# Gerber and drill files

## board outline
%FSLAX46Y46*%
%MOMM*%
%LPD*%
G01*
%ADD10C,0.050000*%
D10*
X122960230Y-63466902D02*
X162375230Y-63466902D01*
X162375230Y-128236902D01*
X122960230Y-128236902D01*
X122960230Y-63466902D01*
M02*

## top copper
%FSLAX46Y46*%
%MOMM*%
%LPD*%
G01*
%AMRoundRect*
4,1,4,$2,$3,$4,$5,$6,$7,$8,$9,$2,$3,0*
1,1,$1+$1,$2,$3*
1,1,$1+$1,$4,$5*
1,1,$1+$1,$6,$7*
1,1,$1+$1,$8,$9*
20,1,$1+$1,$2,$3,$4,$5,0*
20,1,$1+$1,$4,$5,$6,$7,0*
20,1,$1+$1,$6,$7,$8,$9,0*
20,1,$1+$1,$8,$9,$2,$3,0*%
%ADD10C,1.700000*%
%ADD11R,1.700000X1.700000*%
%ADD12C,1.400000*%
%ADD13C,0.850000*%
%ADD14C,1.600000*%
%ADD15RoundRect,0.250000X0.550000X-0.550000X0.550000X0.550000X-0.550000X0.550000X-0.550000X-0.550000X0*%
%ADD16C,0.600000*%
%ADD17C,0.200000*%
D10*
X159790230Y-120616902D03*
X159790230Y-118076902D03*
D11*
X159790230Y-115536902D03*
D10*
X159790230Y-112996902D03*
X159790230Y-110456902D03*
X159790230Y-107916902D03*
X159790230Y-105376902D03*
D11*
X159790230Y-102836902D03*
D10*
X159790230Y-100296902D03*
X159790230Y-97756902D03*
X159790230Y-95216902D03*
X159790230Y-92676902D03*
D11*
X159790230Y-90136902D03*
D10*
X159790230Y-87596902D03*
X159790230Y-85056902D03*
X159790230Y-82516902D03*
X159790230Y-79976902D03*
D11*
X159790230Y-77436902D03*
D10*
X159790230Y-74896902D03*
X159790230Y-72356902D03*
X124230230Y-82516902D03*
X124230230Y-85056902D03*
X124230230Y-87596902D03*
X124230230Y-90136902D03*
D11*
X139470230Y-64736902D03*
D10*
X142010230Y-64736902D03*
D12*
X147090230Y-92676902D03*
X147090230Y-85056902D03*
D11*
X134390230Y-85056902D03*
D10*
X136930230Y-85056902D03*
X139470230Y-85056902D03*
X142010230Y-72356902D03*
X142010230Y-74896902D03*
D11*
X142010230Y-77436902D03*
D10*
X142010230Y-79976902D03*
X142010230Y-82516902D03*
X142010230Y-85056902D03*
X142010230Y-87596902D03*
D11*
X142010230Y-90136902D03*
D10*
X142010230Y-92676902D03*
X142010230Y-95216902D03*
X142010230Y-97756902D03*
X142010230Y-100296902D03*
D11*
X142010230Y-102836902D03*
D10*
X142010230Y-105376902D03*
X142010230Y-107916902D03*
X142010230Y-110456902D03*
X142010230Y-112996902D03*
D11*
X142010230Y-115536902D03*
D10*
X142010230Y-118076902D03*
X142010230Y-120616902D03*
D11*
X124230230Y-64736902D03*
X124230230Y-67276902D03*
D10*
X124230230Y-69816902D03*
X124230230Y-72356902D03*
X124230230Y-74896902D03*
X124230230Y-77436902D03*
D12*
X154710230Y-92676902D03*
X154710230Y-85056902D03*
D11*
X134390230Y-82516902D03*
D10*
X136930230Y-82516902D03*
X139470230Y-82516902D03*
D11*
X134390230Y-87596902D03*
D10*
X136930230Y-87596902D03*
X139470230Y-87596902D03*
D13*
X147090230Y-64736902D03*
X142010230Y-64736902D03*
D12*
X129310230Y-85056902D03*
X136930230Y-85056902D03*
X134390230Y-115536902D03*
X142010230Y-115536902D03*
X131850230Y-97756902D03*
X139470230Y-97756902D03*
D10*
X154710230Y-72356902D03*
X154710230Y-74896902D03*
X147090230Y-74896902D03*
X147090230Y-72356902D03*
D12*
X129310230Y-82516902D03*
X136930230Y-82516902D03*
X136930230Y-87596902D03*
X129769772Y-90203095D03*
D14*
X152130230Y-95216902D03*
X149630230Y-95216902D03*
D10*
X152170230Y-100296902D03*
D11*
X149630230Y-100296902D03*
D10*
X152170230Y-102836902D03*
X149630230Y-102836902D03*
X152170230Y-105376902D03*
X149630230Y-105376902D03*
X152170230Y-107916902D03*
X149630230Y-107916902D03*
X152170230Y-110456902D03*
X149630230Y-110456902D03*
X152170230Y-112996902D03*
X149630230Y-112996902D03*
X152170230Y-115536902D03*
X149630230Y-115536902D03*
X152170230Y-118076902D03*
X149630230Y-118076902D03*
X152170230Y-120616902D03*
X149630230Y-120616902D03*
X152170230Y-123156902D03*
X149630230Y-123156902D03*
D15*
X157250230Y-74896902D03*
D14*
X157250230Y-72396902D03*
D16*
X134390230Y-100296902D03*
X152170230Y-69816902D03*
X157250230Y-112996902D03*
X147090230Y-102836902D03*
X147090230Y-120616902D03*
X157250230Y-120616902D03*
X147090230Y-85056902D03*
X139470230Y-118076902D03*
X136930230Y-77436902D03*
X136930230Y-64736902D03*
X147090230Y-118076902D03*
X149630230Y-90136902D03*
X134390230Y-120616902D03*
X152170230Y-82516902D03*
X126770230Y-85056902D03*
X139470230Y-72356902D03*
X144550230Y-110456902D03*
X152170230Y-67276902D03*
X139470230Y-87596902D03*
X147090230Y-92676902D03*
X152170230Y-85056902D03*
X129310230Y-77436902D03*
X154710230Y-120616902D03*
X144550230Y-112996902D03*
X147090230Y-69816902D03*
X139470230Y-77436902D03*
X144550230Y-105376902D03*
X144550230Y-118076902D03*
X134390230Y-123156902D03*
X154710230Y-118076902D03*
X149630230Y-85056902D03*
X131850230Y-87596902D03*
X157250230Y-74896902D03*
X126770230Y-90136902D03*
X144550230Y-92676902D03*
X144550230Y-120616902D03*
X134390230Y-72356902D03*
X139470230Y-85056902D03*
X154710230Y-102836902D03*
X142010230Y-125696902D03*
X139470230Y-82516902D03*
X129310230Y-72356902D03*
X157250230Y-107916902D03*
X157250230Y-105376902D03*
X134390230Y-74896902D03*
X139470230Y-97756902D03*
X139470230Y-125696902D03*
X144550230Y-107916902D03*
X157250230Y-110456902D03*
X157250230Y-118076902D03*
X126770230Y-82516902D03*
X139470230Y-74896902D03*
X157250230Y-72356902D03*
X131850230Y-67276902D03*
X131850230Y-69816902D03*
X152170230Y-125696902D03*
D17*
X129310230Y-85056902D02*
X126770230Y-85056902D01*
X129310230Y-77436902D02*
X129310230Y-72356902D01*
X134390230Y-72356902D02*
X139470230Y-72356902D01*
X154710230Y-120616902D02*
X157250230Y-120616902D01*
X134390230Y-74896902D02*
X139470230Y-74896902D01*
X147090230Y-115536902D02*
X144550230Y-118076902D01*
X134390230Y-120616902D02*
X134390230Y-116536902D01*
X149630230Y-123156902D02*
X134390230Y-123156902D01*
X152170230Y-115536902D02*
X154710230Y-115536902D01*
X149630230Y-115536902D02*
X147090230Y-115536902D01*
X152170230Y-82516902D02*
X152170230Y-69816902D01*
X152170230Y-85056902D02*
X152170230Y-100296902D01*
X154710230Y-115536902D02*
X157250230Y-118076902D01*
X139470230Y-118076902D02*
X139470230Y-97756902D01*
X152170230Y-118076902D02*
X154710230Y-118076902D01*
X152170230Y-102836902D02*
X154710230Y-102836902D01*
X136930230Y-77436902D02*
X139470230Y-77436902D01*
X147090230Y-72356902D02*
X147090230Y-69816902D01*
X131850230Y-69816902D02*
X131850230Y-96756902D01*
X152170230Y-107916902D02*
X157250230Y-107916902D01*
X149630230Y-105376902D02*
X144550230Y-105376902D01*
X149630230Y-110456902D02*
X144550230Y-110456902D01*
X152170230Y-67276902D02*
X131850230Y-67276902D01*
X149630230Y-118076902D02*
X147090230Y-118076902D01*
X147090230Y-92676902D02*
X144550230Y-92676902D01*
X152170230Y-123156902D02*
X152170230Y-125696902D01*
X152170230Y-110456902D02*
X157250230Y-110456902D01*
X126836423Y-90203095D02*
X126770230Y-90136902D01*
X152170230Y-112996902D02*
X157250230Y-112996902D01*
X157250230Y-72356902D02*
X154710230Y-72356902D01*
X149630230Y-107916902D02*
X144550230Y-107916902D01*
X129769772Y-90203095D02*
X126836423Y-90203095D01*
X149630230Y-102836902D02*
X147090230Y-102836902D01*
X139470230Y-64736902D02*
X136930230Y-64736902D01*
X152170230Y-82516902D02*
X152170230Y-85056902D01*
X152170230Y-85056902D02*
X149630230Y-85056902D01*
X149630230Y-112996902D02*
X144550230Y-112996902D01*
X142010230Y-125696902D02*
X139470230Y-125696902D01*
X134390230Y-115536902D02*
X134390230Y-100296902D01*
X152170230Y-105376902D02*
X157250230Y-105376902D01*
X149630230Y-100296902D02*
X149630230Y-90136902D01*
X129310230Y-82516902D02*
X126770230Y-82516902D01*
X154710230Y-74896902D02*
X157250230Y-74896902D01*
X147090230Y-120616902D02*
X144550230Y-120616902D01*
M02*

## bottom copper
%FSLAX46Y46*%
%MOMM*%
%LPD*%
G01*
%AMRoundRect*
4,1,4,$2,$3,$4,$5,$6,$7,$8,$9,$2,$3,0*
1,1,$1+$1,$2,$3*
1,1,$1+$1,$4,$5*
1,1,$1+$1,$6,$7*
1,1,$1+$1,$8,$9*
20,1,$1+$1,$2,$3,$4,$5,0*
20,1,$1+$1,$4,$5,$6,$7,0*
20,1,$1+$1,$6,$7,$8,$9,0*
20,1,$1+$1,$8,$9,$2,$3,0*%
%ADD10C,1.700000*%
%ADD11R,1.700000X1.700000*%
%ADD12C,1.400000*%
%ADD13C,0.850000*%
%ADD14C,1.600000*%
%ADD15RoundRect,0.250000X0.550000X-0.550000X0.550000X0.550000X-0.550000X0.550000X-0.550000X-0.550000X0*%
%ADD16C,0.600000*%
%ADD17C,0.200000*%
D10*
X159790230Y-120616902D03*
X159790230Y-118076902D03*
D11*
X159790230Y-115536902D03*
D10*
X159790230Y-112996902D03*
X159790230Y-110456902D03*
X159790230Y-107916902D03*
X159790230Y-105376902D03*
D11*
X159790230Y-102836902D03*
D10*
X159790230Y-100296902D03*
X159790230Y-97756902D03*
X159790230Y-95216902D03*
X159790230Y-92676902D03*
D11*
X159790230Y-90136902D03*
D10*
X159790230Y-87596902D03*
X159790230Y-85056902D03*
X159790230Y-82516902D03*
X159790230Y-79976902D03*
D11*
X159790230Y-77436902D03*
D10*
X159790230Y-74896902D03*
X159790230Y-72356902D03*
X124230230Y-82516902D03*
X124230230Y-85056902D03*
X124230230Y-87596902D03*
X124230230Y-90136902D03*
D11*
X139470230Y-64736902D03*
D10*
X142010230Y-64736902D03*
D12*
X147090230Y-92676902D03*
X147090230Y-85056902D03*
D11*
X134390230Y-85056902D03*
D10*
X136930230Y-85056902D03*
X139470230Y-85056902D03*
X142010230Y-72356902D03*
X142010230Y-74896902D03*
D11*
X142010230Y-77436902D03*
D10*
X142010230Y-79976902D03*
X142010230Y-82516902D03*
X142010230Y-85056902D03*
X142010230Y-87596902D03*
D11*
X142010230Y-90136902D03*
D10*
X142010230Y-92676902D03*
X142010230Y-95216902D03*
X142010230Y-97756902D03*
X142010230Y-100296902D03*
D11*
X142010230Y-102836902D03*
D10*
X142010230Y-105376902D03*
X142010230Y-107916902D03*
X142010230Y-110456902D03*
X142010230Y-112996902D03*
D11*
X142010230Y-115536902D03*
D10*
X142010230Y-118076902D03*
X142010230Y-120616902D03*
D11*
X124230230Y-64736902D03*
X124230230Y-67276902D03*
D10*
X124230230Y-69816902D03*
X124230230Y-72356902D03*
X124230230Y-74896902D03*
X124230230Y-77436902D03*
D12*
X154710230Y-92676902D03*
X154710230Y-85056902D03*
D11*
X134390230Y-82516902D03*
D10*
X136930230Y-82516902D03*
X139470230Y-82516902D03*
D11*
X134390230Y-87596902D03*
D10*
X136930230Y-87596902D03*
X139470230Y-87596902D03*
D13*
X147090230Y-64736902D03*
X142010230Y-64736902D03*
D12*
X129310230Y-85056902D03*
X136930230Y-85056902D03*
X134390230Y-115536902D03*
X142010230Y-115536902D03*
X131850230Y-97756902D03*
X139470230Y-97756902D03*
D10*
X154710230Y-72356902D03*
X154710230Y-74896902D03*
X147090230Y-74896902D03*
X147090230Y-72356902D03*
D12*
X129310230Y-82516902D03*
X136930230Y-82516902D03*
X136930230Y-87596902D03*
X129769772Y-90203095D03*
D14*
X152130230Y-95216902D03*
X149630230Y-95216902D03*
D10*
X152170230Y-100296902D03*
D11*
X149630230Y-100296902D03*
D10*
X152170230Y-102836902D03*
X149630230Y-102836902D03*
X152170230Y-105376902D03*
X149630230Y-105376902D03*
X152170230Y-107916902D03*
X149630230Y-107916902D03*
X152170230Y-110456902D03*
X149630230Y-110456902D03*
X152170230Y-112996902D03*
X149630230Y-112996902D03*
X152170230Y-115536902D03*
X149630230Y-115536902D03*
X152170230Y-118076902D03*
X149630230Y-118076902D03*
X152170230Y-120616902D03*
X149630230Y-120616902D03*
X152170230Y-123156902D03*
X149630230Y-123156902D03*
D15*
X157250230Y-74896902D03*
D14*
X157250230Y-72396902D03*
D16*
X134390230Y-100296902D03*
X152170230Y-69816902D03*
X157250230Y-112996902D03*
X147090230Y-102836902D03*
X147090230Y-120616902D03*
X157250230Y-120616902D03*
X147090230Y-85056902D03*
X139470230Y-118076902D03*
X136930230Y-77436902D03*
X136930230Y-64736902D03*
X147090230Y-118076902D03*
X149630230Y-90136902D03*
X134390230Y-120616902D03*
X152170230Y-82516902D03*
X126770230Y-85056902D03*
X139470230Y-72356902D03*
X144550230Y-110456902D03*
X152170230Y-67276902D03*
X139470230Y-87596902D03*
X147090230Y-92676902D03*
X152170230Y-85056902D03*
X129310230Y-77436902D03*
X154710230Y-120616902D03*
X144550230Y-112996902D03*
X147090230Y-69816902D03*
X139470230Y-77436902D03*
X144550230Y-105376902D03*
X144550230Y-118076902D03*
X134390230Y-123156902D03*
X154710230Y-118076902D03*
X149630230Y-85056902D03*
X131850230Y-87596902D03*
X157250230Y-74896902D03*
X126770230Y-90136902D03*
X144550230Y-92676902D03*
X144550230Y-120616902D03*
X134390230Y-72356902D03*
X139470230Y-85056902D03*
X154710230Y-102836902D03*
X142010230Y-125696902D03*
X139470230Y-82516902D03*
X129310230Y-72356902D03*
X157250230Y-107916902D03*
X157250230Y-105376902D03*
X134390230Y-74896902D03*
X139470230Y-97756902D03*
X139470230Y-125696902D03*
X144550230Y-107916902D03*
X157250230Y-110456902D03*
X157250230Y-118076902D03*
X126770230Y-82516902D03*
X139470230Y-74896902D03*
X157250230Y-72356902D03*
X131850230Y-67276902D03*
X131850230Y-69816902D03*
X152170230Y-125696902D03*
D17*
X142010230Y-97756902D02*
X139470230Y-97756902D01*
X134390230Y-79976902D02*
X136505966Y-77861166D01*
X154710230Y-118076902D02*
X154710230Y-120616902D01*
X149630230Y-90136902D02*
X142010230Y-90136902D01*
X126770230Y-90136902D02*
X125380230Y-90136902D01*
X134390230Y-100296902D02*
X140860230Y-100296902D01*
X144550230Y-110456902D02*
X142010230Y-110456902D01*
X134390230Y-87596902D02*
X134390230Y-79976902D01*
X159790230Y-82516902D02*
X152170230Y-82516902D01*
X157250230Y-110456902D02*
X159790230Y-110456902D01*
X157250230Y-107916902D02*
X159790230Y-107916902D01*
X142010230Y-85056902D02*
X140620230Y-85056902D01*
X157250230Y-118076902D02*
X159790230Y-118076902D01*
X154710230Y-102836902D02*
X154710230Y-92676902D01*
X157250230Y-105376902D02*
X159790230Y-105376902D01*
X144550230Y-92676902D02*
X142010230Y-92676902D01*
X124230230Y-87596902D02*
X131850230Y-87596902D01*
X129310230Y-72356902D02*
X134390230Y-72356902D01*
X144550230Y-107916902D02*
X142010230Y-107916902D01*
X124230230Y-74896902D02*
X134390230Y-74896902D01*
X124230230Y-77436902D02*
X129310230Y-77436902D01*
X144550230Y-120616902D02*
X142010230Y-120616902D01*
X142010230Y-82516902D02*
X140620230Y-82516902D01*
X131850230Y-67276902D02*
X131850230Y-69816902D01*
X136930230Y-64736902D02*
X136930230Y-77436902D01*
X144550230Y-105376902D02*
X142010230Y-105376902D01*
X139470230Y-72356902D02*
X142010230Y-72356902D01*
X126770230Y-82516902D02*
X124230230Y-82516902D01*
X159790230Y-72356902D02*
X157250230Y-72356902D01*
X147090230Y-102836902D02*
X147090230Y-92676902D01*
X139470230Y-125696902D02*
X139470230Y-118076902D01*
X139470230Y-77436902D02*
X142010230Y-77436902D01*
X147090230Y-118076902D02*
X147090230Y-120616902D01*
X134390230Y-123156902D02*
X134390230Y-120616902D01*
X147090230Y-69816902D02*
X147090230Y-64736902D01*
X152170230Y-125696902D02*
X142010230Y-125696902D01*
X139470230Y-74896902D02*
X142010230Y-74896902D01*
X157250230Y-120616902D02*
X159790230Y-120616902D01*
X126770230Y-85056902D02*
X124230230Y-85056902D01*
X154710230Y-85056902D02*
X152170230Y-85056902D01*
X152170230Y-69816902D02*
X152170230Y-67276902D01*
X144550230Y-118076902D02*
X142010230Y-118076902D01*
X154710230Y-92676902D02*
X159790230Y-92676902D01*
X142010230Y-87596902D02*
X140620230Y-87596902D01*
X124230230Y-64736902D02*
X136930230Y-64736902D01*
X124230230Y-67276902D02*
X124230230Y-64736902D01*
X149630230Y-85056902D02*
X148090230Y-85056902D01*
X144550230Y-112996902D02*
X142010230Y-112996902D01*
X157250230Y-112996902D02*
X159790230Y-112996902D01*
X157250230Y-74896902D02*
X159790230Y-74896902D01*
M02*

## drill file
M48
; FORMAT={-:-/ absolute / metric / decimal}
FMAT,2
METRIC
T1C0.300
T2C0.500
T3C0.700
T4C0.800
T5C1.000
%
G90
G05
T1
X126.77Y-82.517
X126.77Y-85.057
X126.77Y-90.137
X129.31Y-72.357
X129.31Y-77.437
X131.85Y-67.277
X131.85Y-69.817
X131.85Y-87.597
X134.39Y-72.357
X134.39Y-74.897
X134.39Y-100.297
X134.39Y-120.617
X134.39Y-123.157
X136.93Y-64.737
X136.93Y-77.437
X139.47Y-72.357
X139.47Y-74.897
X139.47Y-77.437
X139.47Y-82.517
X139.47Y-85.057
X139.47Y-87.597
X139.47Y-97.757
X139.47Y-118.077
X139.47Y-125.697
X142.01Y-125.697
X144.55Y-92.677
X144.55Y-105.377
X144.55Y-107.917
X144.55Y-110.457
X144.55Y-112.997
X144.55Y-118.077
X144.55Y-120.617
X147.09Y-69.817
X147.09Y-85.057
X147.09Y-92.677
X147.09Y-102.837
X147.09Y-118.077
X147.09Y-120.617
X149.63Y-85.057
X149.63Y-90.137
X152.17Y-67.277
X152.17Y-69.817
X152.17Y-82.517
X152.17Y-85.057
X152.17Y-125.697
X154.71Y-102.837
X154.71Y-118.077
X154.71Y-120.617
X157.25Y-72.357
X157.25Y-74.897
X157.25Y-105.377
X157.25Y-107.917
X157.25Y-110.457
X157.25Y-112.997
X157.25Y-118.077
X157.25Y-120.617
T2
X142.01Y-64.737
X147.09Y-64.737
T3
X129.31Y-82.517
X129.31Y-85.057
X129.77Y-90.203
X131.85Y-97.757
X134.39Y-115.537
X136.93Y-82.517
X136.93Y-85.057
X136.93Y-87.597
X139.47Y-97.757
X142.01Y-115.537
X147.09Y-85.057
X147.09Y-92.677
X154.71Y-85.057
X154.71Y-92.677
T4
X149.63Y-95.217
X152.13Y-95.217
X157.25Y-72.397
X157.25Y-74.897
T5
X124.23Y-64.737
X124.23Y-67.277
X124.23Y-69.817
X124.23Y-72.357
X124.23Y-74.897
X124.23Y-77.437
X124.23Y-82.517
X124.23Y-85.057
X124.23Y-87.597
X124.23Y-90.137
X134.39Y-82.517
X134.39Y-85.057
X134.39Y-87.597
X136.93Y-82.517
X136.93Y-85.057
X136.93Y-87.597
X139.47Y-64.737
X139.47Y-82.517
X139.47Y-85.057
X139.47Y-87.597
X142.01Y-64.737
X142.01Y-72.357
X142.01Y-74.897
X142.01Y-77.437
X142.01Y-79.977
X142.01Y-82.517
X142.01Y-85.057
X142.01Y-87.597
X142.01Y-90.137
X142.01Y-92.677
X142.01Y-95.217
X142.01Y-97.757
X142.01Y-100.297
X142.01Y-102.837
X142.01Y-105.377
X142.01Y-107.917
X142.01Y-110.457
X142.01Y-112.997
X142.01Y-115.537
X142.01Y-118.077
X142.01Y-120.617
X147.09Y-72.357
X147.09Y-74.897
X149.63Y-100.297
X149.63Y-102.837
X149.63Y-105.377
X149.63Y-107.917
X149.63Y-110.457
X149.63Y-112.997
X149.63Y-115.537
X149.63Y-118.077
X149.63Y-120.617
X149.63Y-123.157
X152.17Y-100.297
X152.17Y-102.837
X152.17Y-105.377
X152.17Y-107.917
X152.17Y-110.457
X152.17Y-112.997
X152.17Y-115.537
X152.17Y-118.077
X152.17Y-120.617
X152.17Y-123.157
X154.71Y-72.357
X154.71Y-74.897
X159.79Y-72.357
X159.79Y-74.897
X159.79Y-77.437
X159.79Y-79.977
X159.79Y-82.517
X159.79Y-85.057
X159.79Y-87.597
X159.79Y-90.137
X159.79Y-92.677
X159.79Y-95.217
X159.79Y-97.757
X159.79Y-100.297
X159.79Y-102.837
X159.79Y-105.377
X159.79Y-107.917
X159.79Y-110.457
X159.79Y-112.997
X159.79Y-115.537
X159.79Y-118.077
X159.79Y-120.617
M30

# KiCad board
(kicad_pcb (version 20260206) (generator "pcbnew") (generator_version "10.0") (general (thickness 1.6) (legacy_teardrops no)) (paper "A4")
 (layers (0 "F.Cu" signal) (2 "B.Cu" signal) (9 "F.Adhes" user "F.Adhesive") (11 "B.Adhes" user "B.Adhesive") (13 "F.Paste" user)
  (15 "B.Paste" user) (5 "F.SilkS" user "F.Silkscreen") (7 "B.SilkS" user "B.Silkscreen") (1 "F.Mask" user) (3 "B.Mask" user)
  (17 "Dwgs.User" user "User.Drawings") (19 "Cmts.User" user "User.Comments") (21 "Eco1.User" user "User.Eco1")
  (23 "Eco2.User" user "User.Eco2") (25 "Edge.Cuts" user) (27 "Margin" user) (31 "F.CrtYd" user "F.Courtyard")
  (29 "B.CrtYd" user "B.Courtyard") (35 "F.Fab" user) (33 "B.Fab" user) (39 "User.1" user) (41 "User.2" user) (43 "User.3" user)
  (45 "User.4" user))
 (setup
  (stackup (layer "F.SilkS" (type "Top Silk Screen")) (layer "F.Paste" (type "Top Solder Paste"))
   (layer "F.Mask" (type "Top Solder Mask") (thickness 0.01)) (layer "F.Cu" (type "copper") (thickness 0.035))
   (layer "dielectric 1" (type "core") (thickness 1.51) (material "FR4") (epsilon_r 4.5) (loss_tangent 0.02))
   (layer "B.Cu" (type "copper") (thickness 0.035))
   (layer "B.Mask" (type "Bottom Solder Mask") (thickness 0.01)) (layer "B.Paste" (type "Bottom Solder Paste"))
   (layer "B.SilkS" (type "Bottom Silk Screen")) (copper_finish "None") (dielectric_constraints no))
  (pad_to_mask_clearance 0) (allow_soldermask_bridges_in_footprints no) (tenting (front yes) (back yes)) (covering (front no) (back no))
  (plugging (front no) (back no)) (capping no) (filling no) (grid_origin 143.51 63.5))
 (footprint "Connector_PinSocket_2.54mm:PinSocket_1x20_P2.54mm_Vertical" (layer "F.Cu") (at 159.79023 72.356902)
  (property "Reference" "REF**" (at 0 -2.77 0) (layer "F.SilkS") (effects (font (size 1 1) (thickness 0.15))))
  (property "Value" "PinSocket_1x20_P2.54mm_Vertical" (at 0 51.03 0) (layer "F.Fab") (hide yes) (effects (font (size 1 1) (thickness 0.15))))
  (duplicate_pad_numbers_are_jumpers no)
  (pad "21" thru_hole circle (at 0 48.26) (size 1.7 1.7) (drill 1) (layers "*.Cu" "*.Mask") (remove_unused_layers no))
  (pad "22" thru_hole circle (at 0 45.72) (size 1.7 1.7) (drill 1) (layers "*.Cu" "*.Mask") (remove_unused_layers no))
  (pad "23" thru_hole rect (at 0 43.18) (size 1.7 1.7) (drill 1) (layers "*.Cu" "*.Mask") (remove_unused_layers no)
   (thermal_bridge_angle 45))
  (pad "24" thru_hole circle (at 0 40.64) (size 1.7 1.7) (drill 1) (layers "*.Cu" "*.Mask") (remove_unused_layers no))
  (pad "25" thru_hole circle (at 0 38.1) (size 1.7 1.7) (drill 1) (layers "*.Cu" "*.Mask") (remove_unused_layers no))
  (pad "26" thru_hole circle (at 0 35.56) (size 1.7 1.7) (drill 1) (layers "*.Cu" "*.Mask") (remove_unused_layers no))
  (pad "27" thru_hole circle (at 0 33.02) (size 1.7 1.7) (drill 1) (layers "*.Cu" "*.Mask") (remove_unused_layers no))
  (pad "28" thru_hole rect (at 0 30.48) (size 1.7 1.7) (drill 1) (layers "*.Cu" "*.Mask") (remove_unused_layers no)
   (thermal_bridge_angle 45))
  (pad "29" thru_hole circle (at 0 27.94) (size 1.7 1.7) (drill 1) (layers "*.Cu" "*.Mask") (remove_unused_layers no))
  (pad "30" thru_hole circle (at 0 25.4) (size 1.7 1.7) (drill 1) (layers "*.Cu" "*.Mask") (remove_unused_layers no))
  (pad "31" thru_hole circle (at 0 22.86) (size 1.7 1.7) (drill 1) (layers "*.Cu" "*.Mask") (remove_unused_layers no))
  (pad "32" thru_hole circle (at 0 20.32) (size 1.7 1.7) (drill 1) (layers "*.Cu" "*.Mask") (remove_unused_layers no))
  (pad "33" thru_hole rect (at 0 17.78) (size 1.7 1.7) (drill 1) (layers "*.Cu" "*.Mask") (remove_unused_layers no)
   (thermal_bridge_angle 45))
  (pad "34" thru_hole circle (at 0 15.24) (size 1.7 1.7) (drill 1) (layers "*.Cu" "*.Mask") (remove_unused_layers no))
  (pad "35" thru_hole circle (at 0 12.7) (size 1.7 1.7) (drill 1) (layers "*.Cu" "*.Mask") (remove_unused_layers no))
  (pad "36" thru_hole circle (at 0 10.16) (size 1.7 1.7) (drill 1) (layers "*.Cu" "*.Mask") (remove_unused_layers no))
  (pad "37" thru_hole circle (at 0 7.62) (size 1.7 1.7) (drill 1) (layers "*.Cu" "*.Mask") (remove_unused_layers no))
  (pad "38" thru_hole rect (at 0 5.08) (size 1.7 1.7) (drill 1) (layers "*.Cu" "*.Mask") (remove_unused_layers no) (thermal_bridge_angle 45))
  (pad "39" thru_hole circle (at 0 2.54) (size 1.7 1.7) (drill 1) (layers "*.Cu" "*.Mask") (remove_unused_layers no))
  (pad "40" thru_hole circle (at 0 0) (size 1.7 1.7) (drill 1) (layers "*.Cu" "*.Mask") (remove_unused_layers no) (thermal_bridge_angle 90)))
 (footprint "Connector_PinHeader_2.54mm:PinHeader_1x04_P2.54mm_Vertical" (layer "F.Cu") (at 124.23023 82.516902)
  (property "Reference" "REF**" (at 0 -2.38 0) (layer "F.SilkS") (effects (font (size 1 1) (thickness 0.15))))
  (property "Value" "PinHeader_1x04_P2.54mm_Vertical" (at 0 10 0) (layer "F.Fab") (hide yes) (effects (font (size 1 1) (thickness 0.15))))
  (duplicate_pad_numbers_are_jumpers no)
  (pad "1" thru_hole circle (at 0 0) (size 1.7 1.7) (drill 1) (layers "*.Cu" "*.Mask") (remove_unused_layers no) (thermal_bridge_angle 90))
  (pad "2" thru_hole circle (at 0 2.54) (size 1.7 1.7) (drill 1) (layers "*.Cu" "*.Mask") (remove_unused_layers no))
  (pad "3" thru_hole circle (at 0 5.08) (size 1.7 1.7) (drill 1) (layers "*.Cu" "*.Mask") (remove_unused_layers no))
  (pad "4" thru_hole circle (at 0 7.62) (size 1.7 1.7) (drill 1) (layers "*.Cu" "*.Mask") (remove_unused_layers no)))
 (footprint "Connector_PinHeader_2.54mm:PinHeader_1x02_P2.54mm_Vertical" (layer "F.Cu") (at 139.47023 64.736902 90)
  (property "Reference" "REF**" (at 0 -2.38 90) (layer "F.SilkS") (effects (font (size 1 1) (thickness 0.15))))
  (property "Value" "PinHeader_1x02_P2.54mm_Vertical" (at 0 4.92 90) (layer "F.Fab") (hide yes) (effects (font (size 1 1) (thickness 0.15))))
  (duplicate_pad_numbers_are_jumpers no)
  (pad "1" thru_hole rect (at 0 0 90) (size 1.7 1.7) (drill 1) (layers "*.Cu" "*.Mask") (remove_unused_layers no))
  (pad "2" thru_hole circle (at 0 2.54 90) (size 1.7 1.7) (drill 1) (layers "*.Cu" "*.Mask") (remove_unused_layers no)))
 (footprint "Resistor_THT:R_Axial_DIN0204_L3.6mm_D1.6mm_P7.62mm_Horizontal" (layer "F.Cu") (at 147.09023 92.676902 90)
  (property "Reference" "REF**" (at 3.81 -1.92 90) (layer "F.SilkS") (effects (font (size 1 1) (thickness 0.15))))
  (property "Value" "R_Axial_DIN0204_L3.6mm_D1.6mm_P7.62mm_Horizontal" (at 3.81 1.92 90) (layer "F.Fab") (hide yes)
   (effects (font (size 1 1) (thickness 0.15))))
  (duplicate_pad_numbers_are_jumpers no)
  (pad "1" thru_hole circle (at 0 0 90) (size 1.4 1.4) (drill 0.7) (layers "*.Cu" "*.Mask") (remove_unused_layers no))
  (pad "2" thru_hole circle (at 7.62 0 90) (size 1.4 1.4) (drill 0.7) (layers "*.Cu" "*.Mask") (remove_unused_layers no)))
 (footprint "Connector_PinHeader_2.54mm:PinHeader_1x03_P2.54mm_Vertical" (layer "F.Cu") (at 134.39023 85.056902 90)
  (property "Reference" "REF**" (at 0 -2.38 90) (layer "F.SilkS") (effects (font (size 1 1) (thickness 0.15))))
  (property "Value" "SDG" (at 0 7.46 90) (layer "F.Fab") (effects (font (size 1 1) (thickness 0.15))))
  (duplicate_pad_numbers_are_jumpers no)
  (pad "1" thru_hole rect (at 0 0 90) (size 1.7 1.7) (drill 1) (layers "*.Cu" "*.Mask") (remove_unused_layers no))
  (pad "2" thru_hole circle (at 0 2.54 90) (size 1.7 1.7) (drill 1) (layers "*.Cu" "*.Mask") (remove_unused_layers no))
  (pad "3" thru_hole circle (at 0 5.08 90) (size 1.7 1.7) (drill 1) (layers "*.Cu" "*.Mask") (remove_unused_layers no)))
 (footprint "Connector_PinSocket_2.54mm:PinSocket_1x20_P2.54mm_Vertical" (layer "F.Cu") (at 142.01023 72.356902)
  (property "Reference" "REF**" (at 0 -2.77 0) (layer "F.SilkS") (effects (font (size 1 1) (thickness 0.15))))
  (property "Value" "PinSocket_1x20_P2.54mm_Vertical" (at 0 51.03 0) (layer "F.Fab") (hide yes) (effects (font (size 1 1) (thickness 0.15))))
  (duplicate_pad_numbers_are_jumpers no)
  (pad "1" thru_hole circle (at 0 0) (size 1.7 1.7) (drill 1) (layers "*.Cu" "*.Mask") (remove_unused_layers no) (thermal_bridge_angle 90))
  (pad "2" thru_hole circle (at 0 2.54) (size 1.7 1.7) (drill 1) (layers "*.Cu" "*.Mask") (remove_unused_layers no))
  (pad "3" thru_hole rect (at 0 5.08) (size 1.7 1.7) (drill 1) (layers "*.Cu" "*.Mask") (remove_unused_layers no) (thermal_bridge_angle 45))
  (pad "4" thru_hole circle (at 0 7.62) (size 1.7 1.7) (drill 1) (layers "*.Cu" "*.Mask") (remove_unused_layers no))
  (pad "5" thru_hole circle (at 0 10.16) (size 1.7 1.7) (drill 1) (layers "*.Cu" "*.Mask") (remove_unused_layers no))
  (pad "6" thru_hole circle (at 0 12.7) (size 1.7 1.7) (drill 1) (layers "*.Cu" "*.Mask") (remove_unused_layers no))
  (pad "7" thru_hole circle (at 0 15.24) (size 1.7 1.7) (drill 1) (layers "*.Cu" "*.Mask") (remove_unused_layers no))
  (pad "8" thru_hole rect (at 0 17.78) (size 1.7 1.7) (drill 1) (layers "*.Cu" "*.Mask") (remove_unused_layers no) (thermal_bridge_angle 45))
  (pad "9" thru_hole circle (at 0 20.32) (size 1.7 1.7) (drill 1) (layers "*.Cu" "*.Mask") (remove_unused_layers no))
  (pad "10" thru_hole circle (at 0 22.86) (size 1.7 1.7) (drill 1) (layers "*.Cu" "*.Mask") (remove_unused_layers no))
  (pad "11" thru_hole circle (at 0 25.4) (size 1.7 1.7) (drill 1) (layers "*.Cu" "*.Mask") (remove_unused_layers no))
  (pad "12" thru_hole circle (at 0 27.94) (size 1.7 1.7) (drill 1) (layers "*.Cu" "*.Mask") (remove_unused_layers no))
  (pad "13" thru_hole rect (at 0 30.48) (size 1.7 1.7) (drill 1) (layers "*.Cu" "*.Mask") (remove_unused_layers no)
   (thermal_bridge_angle 45))
  (pad "14" thru_hole circle (at 0 33.02) (size 1.7 1.7) (drill 1) (layers "*.Cu" "*.Mask") (remove_unused_layers no))
  (pad "15" thru_hole circle (at 0 35.56) (size 1.7 1.7) (drill 1) (layers "*.Cu" "*.Mask") (remove_unused_layers no))
  (pad "16" thru_hole circle (at 0 38.1) (size 1.7 1.7) (drill 1) (layers "*.Cu" "*.Mask") (remove_unused_layers no))
  (pad "17" thru_hole circle (at 0 40.64) (size 1.7 1.7) (drill 1) (layers "*.Cu" "*.Mask") (remove_unused_layers no))
  (pad "18" thru_hole rect (at 0 43.18) (size 1.7 1.7) (drill 1) (layers "*.Cu" "*.Mask") (remove_unused_layers no)
   (thermal_bridge_angle 45))
  (pad "19" thru_hole circle (at 0 45.72) (size 1.7 1.7) (drill 1) (layers "*.Cu" "*.Mask") (remove_unused_layers no))
  (pad "20" thru_hole circle (at 0 48.26) (size 1.7 1.7) (drill 1) (layers "*.Cu" "*.Mask") (remove_unused_layers no)))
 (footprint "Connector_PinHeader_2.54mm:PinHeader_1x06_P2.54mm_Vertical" (layer "F.Cu") (at 124.23023 64.736902)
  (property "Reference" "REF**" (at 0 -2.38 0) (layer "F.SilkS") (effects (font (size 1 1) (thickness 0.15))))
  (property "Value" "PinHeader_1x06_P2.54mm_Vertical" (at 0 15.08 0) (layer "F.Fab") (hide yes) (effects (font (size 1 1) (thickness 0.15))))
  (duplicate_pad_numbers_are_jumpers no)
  (pad "1" thru_hole rect (at 0 0) (size 1.7 1.7) (drill 1) (layers "*.Cu" "*.Mask") (remove_unused_layers no))
  (pad "2" thru_hole rect (at 0 2.54) (size 1.7 1.7) (drill 1) (layers "*.Cu" "*.Mask") (remove_unused_layers no) (thermal_bridge_angle 45))
  (pad "3" thru_hole circle (at 0 5.08) (size 1.7 1.7) (drill 1) (layers "*.Cu" "*.Mask") (remove_unused_layers no))
  (pad "4" thru_hole circle (at 0 7.62) (size 1.7 1.7) (drill 1) (layers "*.Cu" "*.Mask") (remove_unused_layers no))
  (pad "5" thru_hole circle (at 0 10.16) (size 1.7 1.7) (drill 1) (layers "*.Cu" "*.Mask") (remove_unused_layers no))
  (pad "6" thru_hole circle (at 0 12.7) (size 1.7 1.7) (drill 1) (layers "*.Cu" "*.Mask") (remove_unused_layers no)))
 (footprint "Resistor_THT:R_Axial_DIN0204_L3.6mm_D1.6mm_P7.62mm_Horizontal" (layer "F.Cu") (at 154.71023 92.676902 90)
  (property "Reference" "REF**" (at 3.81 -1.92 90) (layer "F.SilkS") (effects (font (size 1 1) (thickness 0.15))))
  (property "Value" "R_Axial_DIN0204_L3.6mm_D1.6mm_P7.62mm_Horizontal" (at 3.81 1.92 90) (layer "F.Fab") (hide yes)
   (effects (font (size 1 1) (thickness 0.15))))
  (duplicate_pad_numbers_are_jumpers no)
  (pad "1" thru_hole circle (at 0 0 90) (size 1.4 1.4) (drill 0.7) (layers "*.Cu" "*.Mask") (remove_unused_layers no))
  (pad "2" thru_hole circle (at 7.62 0 90) (size 1.4 1.4) (drill 0.7) (layers "*.Cu" "*.Mask") (remove_unused_layers no)))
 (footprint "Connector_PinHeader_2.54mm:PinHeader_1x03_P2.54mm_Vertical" (layer "F.Cu") (at 134.39023 82.516902 90)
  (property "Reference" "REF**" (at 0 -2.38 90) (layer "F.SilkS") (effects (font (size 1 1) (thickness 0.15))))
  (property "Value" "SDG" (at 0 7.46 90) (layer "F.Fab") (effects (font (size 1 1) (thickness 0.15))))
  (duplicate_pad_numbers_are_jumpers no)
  (pad "1" thru_hole rect (at 0 0 90) (size 1.7 1.7) (drill 1) (layers "*.Cu" "*.Mask") (remove_unused_layers no))
  (pad "2" thru_hole circle (at 0 2.54 90) (size 1.7 1.7) (drill 1) (layers "*.Cu" "*.Mask") (remove_unused_layers no))
  (pad "3" thru_hole circle (at 0 5.08 90) (size 1.7 1.7) (drill 1) (layers "*.Cu" "*.Mask") (remove_unused_layers no)))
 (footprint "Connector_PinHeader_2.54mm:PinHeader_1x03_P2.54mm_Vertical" (layer "F.Cu") (at 134.39023 87.596902 90)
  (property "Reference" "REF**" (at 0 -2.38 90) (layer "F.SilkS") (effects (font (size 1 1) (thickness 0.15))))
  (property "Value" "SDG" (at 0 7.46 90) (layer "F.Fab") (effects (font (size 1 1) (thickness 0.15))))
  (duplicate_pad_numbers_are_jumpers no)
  (pad "1" thru_hole rect (at 0 0 90) (size 1.7 1.7) (drill 1) (layers "*.Cu" "*.Mask") (remove_unused_layers no))
  (pad "2" thru_hole circle (at 0 2.54 90) (size 1.7 1.7) (drill 1) (layers "*.Cu" "*.Mask") (remove_unused_layers no))
  (pad "3" thru_hole circle (at 0 5.08 90) (size 1.7 1.7) (drill 1) (layers "*.Cu" "*.Mask") (remove_unused_layers no)))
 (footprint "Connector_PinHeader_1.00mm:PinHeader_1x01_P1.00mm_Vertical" (layer "B.Cu") (at 147.09023 64.736902 180)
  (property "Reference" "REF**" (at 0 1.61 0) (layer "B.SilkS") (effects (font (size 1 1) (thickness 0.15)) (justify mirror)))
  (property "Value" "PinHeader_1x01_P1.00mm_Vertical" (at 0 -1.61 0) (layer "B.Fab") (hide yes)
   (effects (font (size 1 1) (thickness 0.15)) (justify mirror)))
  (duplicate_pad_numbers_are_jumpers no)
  (pad "1" thru_hole circle (at 0 0 180) (size 0.85 0.85) (drill 0.5) (layers "*.Cu" "*.Mask") (remove_unused_layers no)
   (thermal_bridge_angle 90))
  (pad "2" thru_hole circle (at 5.08 0 180) (size 0.85 0.85) (drill 0.5) (layers "*.Cu" "*.Mask") (remove_unused_layers no)
   (thermal_bridge_angle 90)))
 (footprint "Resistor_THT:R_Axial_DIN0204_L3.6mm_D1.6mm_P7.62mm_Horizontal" (layer "B.Cu") (at 129.31023 85.056902)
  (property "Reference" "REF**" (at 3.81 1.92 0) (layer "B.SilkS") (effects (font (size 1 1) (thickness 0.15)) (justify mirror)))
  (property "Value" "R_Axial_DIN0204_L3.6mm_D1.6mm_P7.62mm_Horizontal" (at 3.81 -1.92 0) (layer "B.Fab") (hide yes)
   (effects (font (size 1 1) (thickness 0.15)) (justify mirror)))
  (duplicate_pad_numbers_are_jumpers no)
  (pad "1" thru_hole circle (at 0 0) (size 1.4 1.4) (drill 0.7) (layers "*.Cu" "*.Mask") (remove_unused_layers no))
  (pad "2" thru_hole circle (at 7.62 0) (size 1.4 1.4) (drill 0.7) (layers "*.Cu" "*.Mask") (remove_unused_layers no)))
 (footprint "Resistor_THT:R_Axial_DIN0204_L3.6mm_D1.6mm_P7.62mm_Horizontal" (layer "B.Cu") (at 134.39023 115.536902)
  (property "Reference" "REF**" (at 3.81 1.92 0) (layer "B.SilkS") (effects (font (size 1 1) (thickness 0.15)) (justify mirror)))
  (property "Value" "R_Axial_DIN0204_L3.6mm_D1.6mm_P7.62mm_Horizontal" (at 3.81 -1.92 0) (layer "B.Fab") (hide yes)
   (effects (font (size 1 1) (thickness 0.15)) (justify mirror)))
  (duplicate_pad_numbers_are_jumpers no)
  (pad "1" thru_hole circle (at 0 0) (size 1.4 1.4) (drill 0.7) (layers "*.Cu" "*.Mask") (remove_unused_layers no))
  (pad "2" thru_hole circle (at 7.62 0) (size 1.4 1.4) (drill 0.7) (layers "*.Cu" "*.Mask") (remove_unused_layers no)))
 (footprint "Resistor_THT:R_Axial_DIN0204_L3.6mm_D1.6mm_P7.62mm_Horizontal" (layer "B.Cu") (at 131.85023 97.756902)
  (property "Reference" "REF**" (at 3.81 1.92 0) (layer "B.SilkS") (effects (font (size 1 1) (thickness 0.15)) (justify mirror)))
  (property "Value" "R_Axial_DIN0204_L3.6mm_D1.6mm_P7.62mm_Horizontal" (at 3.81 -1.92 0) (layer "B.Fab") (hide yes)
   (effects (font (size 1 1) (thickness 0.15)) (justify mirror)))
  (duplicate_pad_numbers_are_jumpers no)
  (pad "1" thru_hole circle (at 0 0) (size 1.4 1.4) (drill 0.7) (layers "*.Cu" "*.Mask") (remove_unused_layers no))
  (pad "2" thru_hole circle (at 7.62 0) (size 1.4 1.4) (drill 0.7) (layers "*.Cu" "*.Mask") (remove_unused_layers no)))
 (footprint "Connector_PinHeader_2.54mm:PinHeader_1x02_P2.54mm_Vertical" (layer "B.Cu") (at 154.71023 72.356902 180)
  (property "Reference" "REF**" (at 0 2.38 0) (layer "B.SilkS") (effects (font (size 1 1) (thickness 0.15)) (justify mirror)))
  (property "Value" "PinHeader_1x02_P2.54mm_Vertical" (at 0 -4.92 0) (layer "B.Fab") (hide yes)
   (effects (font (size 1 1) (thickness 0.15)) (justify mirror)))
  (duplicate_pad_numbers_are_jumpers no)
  (pad "1" thru_hole circle (at 0 0 180) (size 1.7 1.7) (drill 1) (layers "*.Cu" "*.Mask") (remove_unused_layers no)
   (thermal_bridge_angle 90))
  (pad "2" thru_hole circle (at 0 -2.54 180) (size 1.7 1.7) (drill 1) (layers "*.Cu" "*.Mask") (remove_unused_layers no))
  (pad "3" thru_hole circle (at 7.62 -2.54 180) (size 1.7 1.7) (drill 1) (layers "*.Cu" "*.Mask") (remove_unused_layers no))
  (pad "3" thru_hole circle (at 7.62 0 180) (size 1.7 1.7) (drill 1) (layers "*.Cu" "*.Mask") (remove_unused_layers no)
   (thermal_bridge_angle 90)))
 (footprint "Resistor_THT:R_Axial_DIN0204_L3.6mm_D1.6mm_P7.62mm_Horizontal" (layer "B.Cu") (at 129.31023 82.516902)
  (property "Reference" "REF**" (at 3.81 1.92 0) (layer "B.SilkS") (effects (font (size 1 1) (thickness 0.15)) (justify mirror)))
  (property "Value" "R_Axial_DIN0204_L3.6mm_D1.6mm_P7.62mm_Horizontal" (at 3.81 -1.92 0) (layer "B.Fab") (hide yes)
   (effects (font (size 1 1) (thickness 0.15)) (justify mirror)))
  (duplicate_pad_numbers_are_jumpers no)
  (pad "1" thru_hole circle (at 0 0) (size 1.4 1.4) (drill 0.7) (layers "*.Cu" "*.Mask") (remove_unused_layers no))
  (pad "2" thru_hole circle (at 7.62 0) (size 1.4 1.4) (drill 0.7) (layers "*.Cu" "*.Mask") (remove_unused_layers no)))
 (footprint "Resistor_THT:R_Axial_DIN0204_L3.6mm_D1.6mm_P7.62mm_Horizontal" (layer "B.Cu") (at 136.93023 87.596902 -160)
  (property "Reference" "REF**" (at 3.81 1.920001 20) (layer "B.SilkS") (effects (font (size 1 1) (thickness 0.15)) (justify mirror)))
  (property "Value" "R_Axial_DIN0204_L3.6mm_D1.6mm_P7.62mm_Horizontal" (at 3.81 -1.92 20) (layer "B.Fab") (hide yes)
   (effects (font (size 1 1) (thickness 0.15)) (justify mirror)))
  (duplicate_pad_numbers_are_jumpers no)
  (pad "1" thru_hole circle (at 0 0 200) (size 1.4 1.4) (drill 0.7) (layers "*.Cu" "*.Mask") (remove_unused_layers no))
  (pad "2" thru_hole circle (at 7.62 0.000001 200) (size 1.4 1.4) (drill 0.7) (layers "*.Cu" "*.Mask") (remove_unused_layers no)))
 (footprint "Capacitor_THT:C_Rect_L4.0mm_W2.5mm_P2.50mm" (layer "B.Cu") (at 152.13023 95.216902 180)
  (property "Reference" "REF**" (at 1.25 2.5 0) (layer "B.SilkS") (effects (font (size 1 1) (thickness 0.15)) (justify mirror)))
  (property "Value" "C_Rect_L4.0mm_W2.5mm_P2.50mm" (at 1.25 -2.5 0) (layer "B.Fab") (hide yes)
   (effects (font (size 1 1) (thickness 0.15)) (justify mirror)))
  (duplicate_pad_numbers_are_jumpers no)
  (pad "1" thru_hole circle (at 0 0 180) (size 1.6 1.6) (drill 0.8) (layers "*.Cu" "*.Mask") (remove_unused_layers no))
  (pad "2" thru_hole circle (at 2.5 0 180) (size 1.6 1.6) (drill 0.8) (layers "*.Cu" "*.Mask") (remove_unused_layers no)))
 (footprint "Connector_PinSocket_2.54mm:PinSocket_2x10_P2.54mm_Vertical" (layer "B.Cu") (at 149.63023 100.296902 180)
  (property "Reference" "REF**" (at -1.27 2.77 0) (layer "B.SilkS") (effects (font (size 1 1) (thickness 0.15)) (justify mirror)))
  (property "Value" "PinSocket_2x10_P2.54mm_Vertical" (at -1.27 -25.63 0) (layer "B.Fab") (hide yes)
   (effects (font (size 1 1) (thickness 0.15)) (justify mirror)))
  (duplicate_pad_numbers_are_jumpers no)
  (pad "1" thru_hole circle (at -2.54 0 180) (size 1.7 1.7) (drill 1) (layers "*.Cu" "*.Mask") (remove_unused_layers no))
  (pad "2" thru_hole rect (at 0 0 180) (size 1.7 1.7) (drill 1) (layers "*.Cu" "*.Mask") (remove_unused_layers no))
  (pad "3" thru_hole circle (at -2.54 -2.54 180) (size 1.7 1.7) (drill 1) (layers "*.Cu" "*.Mask") (remove_unused_layers no))
  (pad "4" thru_hole circle (at 0 -2.54 180) (size 1.7 1.7) (drill 1) (layers "*.Cu" "*.Mask") (remove_unused_layers no))
  (pad "5" thru_hole circle (at -2.54 -5.08 180) (size 1.7 1.7) (drill 1) (layers "*.Cu" "*.Mask") (remove_unused_layers no))
  (pad "6" thru_hole circle (at 0 -5.08 180) (size 1.7 1.7) (drill 1) (layers "*.Cu" "*.Mask") (remove_unused_layers no))
  (pad "7" thru_hole circle (at -2.54 -7.62 180) (size 1.7 1.7) (drill 1) (layers "*.Cu" "*.Mask") (remove_unused_layers no))
  (pad "8" thru_hole circle (at 0 -7.62 180) (size 1.7 1.7) (drill 1) (layers "*.Cu" "*.Mask") (remove_unused_layers no))
  (pad "9" thru_hole circle (at -2.54 -10.16 180) (size 1.7 1.7) (drill 1) (layers "*.Cu" "*.Mask") (remove_unused_layers no))
  (pad "10" thru_hole circle (at 0 -10.16 180) (size 1.7 1.7) (drill 1) (layers "*.Cu" "*.Mask") (remove_unused_layers no))
  (pad "11" thru_hole circle (at -2.54 -12.7 180) (size 1.7 1.7) (drill 1) (layers "*.Cu" "*.Mask") (remove_unused_layers no))
  (pad "12" thru_hole circle (at 0 -12.7 180) (size 1.7 1.7) (drill 1) (layers "*.Cu" "*.Mask") (remove_unused_layers no))
  (pad "13" thru_hole circle (at -2.54 -15.24 180) (size 1.7 1.7) (drill 1) (layers "*.Cu" "*.Mask") (remove_unused_layers no))
  (pad "14" thru_hole circle (at 0 -15.24 180) (size 1.7 1.7) (drill 1) (layers "*.Cu" "*.Mask") (remove_unused_layers no))
  (pad "15" thru_hole circle (at -2.54 -17.78 180) (size 1.7 1.7) (drill 1) (layers "*.Cu" "*.Mask") (remove_unused_layers no))
  (pad "16" thru_hole circle (at 0 -17.78 180) (size 1.7 1.7) (drill 1) (layers "*.Cu" "*.Mask") (remove_unused_layers no))
  (pad "17" thru_hole circle (at -2.54 -20.32 180) (size 1.7 1.7) (drill 1) (layers "*.Cu" "*.Mask") (remove_unused_layers no))
  (pad "18" thru_hole circle (at 0 -20.32 180) (size 1.7 1.7) (drill 1) (layers "*.Cu" "*.Mask") (remove_unused_layers no))
  (pad "19" thru_hole circle (at -2.54 -22.86 180) (size 1.7 1.7) (drill 1) (layers "*.Cu" "*.Mask") (remove_unused_layers no))
  (pad "20" thru_hole circle (at 0 -22.86 180) (size 1.7 1.7) (drill 1) (layers "*.Cu" "*.Mask") (remove_unused_layers no)))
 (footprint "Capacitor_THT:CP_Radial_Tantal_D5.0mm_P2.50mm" (layer "B.Cu") (at 157.25023 74.896902 90)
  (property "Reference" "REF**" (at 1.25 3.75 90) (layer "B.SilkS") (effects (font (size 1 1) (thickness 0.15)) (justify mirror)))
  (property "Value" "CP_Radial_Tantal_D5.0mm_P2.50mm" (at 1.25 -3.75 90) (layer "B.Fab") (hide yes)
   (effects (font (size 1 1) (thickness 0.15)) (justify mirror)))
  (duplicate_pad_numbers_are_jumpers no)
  (pad "1" thru_hole roundrect (at 0 0 90) (size 1.6 1.6) (drill 0.8) (layers "*.Cu" "*.Mask") (remove_unused_layers no)
   (roundrect_rratio 0.15625))
  (pad "2" thru_hole circle (at 2.5 0 90) (size 1.6 1.6) (drill 0.8) (layers "*.Cu" "*.Mask") (remove_unused_layers no)))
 (gr_rect (start 122.96023 63.466902) (end 162.37523 128.236902) (stroke (width 0.05) (type solid)) (fill no) (layer "Edge.Cuts"))
 (segment (start 129.31023 85.056902) (end 126.77023 85.056902) (width 0.2) (layer "F.Cu") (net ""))
 (segment (start 129.31023 77.436902) (end 129.31023 72.356902) (width 0.2) (layer "F.Cu") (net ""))
 (segment (start 134.39023 72.356902) (end 139.47023 72.356902) (width 0.2) (layer "F.Cu") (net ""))
 (segment (start 154.71023 120.616902) (end 157.25023 120.616902) (width 0.2) (layer "F.Cu") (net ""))
 (segment (start 134.39023 74.896902) (end 139.47023 74.896902) (width 0.2) (layer "F.Cu") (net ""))
 (segment (start 147.09023 115.536902) (end 144.55023 118.076902) (width 0.2) (layer "F.Cu") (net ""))
 (segment (start 134.39023 120.616902) (end 134.39023 116.536902) (width 0.2) (layer "F.Cu") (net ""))
 (segment (start 149.63023 123.156902) (end 134.39023 123.156902) (width 0.2) (layer "F.Cu") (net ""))
 (segment (start 152.17023 115.536902) (end 154.71023 115.536902) (width 0.2) (layer "F.Cu") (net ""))
 (segment (start 149.63023 115.536902) (end 147.09023 115.536902) (width 0.2) (layer "F.Cu") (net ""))
 (segment (start 152.17023 82.516902) (end 152.17023 69.816902) (width 0.2) (layer "F.Cu") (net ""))
 (segment (start 152.17023 85.056902) (end 152.17023 100.296902) (width 0.2) (layer "F.Cu") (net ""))
 (segment (start 154.71023 115.536902) (end 157.25023 118.076902) (width 0.2) (layer "F.Cu") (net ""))
 (segment (start 139.47023 118.076902) (end 139.47023 97.756902) (width 0.2) (layer "F.Cu") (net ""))
 (segment (start 152.17023 118.076902) (end 154.71023 118.076902) (width 0.2) (layer "F.Cu") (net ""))
 (segment (start 152.17023 102.836902) (end 154.71023 102.836902) (width 0.2) (layer "F.Cu") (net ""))
 (segment (start 136.93023 77.436902) (end 139.47023 77.436902) (width 0.2) (layer "F.Cu") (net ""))
 (segment (start 147.09023 72.356902) (end 147.09023 69.816902) (width 0.2) (layer "F.Cu") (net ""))
 (segment (start 131.85023 69.816902) (end 131.85023 96.756902) (width 0.2) (layer "F.Cu") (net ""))
 (segment (start 152.17023 107.916902) (end 157.25023 107.916902) (width 0.2) (layer "F.Cu") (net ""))
 (segment (start 149.63023 105.376902) (end 144.55023 105.376902) (width 0.2) (layer "F.Cu") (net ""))
 (segment (start 149.63023 110.456902) (end 144.55023 110.456902) (width 0.2) (layer "F.Cu") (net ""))
 (segment (start 152.17023 67.276902) (end 131.85023 67.276902) (width 0.2) (layer "F.Cu") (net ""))
 (segment (start 149.63023 118.076902) (end 147.09023 118.076902) (width 0.2) (layer "F.Cu") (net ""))
 (segment (start 147.09023 92.676902) (end 144.55023 92.676902) (width 0.2) (layer "F.Cu") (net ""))
 (segment (start 152.17023 123.156902) (end 152.17023 125.696902) (width 0.2) (layer "F.Cu") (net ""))
 (segment (start 152.17023 110.456902) (end 157.25023 110.456902) (width 0.2) (layer "F.Cu") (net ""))
 (segment (start 126.836423 90.203095) (end 126.77023 90.136902) (width 0.2) (layer "F.Cu") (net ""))
 (segment (start 152.17023 112.996902) (end 157.25023 112.996902) (width 0.2) (layer "F.Cu") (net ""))
 (segment (start 157.25023 72.356902) (end 154.71023 72.356902) (width 0.2) (layer "F.Cu") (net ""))
 (segment (start 149.63023 107.916902) (end 144.55023 107.916902) (width 0.2) (layer "F.Cu") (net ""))
 (segment (start 129.769772 90.203095) (end 126.836423 90.203095) (width 0.2) (layer "F.Cu") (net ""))
 (segment (start 149.63023 102.836902) (end 147.09023 102.836902) (width 0.2) (layer "F.Cu") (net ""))
 (segment (start 139.47023 64.736902) (end 136.93023 64.736902) (width 0.2) (layer "F.Cu") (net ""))
 (segment (start 152.17023 82.516902) (end 152.17023 85.056902) (width 0.2) (layer "F.Cu") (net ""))
 (segment (start 152.17023 85.056902) (end 149.63023 85.056902) (width 0.2) (layer "F.Cu") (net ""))
 (segment (start 149.63023 112.996902) (end 144.55023 112.996902) (width 0.2) (layer "F.Cu") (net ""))
 (segment (start 142.01023 125.696902) (end 139.47023 125.696902) (width 0.2) (layer "F.Cu") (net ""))
 (segment (start 134.39023 115.536902) (end 134.39023 100.296902) (width 0.2) (layer "F.Cu") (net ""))
 (segment (start 152.17023 105.376902) (end 157.25023 105.376902) (width 0.2) (layer "F.Cu") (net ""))
 (segment (start 149.63023 100.296902) (end 149.63023 90.136902) (width 0.2) (layer "F.Cu") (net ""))
 (segment (start 129.31023 82.516902) (end 126.77023 82.516902) (width 0.2) (layer "F.Cu") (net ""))
 (segment (start 154.71023 74.896902) (end 157.25023 74.896902) (width 0.2) (layer "F.Cu") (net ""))
 (segment (start 147.09023 120.616902) (end 144.55023 120.616902) (width 0.2) (layer "F.Cu") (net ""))
 (via (at 134.39023 100.296902) (size 0.6) (drill 0.3) (layers "F.Cu" "B.Cu") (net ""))
 (via (at 152.17023 69.816902) (size 0.6) (drill 0.3) (layers "F.Cu" "B.Cu") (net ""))
 (via (at 157.25023 112.996902) (size 0.6) (drill 0.3) (layers "F.Cu" "B.Cu") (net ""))
 (via (at 147.09023 102.836902) (size 0.6) (drill 0.3) (layers "F.Cu" "B.Cu") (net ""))
 (via (at 147.09023 120.616902) (size 0.6) (drill 0.3) (layers "F.Cu" "B.Cu") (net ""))
 (via (at 157.25023 120.616902) (size 0.6) (drill 0.3) (layers "F.Cu" "B.Cu") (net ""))
 (via (at 147.09023 85.056902) (size 0.6) (drill 0.3) (layers "F.Cu" "B.Cu") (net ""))
 (via (at 139.47023 118.076902) (size 0.6) (drill 0.3) (layers "F.Cu" "B.Cu") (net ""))
 (via (at 136.93023 77.436902) (size 0.6) (drill 0.3) (layers "F.Cu" "B.Cu") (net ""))
 (via (at 136.93023 64.736902) (size 0.6) (drill 0.3) (layers "F.Cu" "B.Cu") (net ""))
 (via (at 147.09023 118.076902) (size 0.6) (drill 0.3) (layers "F.Cu" "B.Cu") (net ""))
 (via (at 149.63023 90.136902) (size 0.6) (drill 0.3) (layers "F.Cu" "B.Cu") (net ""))
 (via (at 134.39023 120.616902) (size 0.6) (drill 0.3) (layers "F.Cu" "B.Cu") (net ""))
 (via (at 152.17023 82.516902) (size 0.6) (drill 0.3) (layers "F.Cu" "B.Cu") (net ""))
 (via (at 126.77023 85.056902) (size 0.6) (drill 0.3) (layers "F.Cu" "B.Cu") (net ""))
 (via (at 139.47023 72.356902) (size 0.6) (drill 0.3) (layers "F.Cu" "B.Cu") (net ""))
 (via (at 144.55023 110.456902) (size 0.6) (drill 0.3) (layers "F.Cu" "B.Cu") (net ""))
 (via (at 152.17023 67.276902) (size 0.6) (drill 0.3) (layers "F.Cu" "B.Cu") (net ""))
 (via (at 139.47023 87.596902) (size 0.6) (drill 0.3) (layers "F.Cu" "B.Cu") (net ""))
 (via (at 147.09023 92.676902) (size 0.6) (drill 0.3) (layers "F.Cu" "B.Cu") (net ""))
 (via (at 152.17023 85.056902) (size 0.6) (drill 0.3) (layers "F.Cu" "B.Cu") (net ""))
 (via (at 129.31023 77.436902) (size 0.6) (drill 0.3) (layers "F.Cu" "B.Cu") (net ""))
 (via (at 154.71023 120.616902) (size 0.6) (drill 0.3) (layers "F.Cu" "B.Cu") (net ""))
 (via (at 144.55023 112.996902) (size 0.6) (drill 0.3) (layers "F.Cu" "B.Cu") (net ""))
 (via (at 147.09023 69.816902) (size 0.6) (drill 0.3) (layers "F.Cu" "B.Cu") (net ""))
 (via (at 139.47023 77.436902) (size 0.6) (drill 0.3) (layers "F.Cu" "B.Cu") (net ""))
 (via (at 144.55023 105.376902) (size 0.6) (drill 0.3) (layers "F.Cu" "B.Cu") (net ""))
 (via (at 144.55023 118.076902) (size 0.6) (drill 0.3) (layers "F.Cu" "B.Cu") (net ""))
 (via (at 134.39023 123.156902) (size 0.6) (drill 0.3) (layers "F.Cu" "B.Cu") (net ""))
 (via (at 154.71023 118.076902) (size 0.6) (drill 0.3) (layers "F.Cu" "B.Cu") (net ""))
 (via (at 149.63023 85.056902) (size 0.6) (drill 0.3) (layers "F.Cu" "B.Cu") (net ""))
 (via (at 131.85023 87.596902) (size 0.6) (drill 0.3) (layers "F.Cu" "B.Cu") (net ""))
 (via (at 157.25023 74.896902) (size 0.6) (drill 0.3) (layers "F.Cu" "B.Cu") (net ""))
 (via (at 126.77023 90.136902) (size 0.6) (drill 0.3) (layers "F.Cu" "B.Cu") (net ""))
 (via (at 144.55023 92.676902) (size 0.6) (drill 0.3) (layers "F.Cu" "B.Cu") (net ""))
 (via (at 144.55023 120.616902) (size 0.6) (drill 0.3) (layers "F.Cu" "B.Cu") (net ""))
 (via (at 134.39023 72.356902) (size 0.6) (drill 0.3) (layers "F.Cu" "B.Cu") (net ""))
 (via (at 139.47023 85.056902) (size 0.6) (drill 0.3) (layers "F.Cu" "B.Cu") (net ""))
 (via (at 154.71023 102.836902) (size 0.6) (drill 0.3) (layers "F.Cu" "B.Cu") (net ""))
 (via (at 142.01023 125.696902) (size 0.6) (drill 0.3) (layers "F.Cu" "B.Cu") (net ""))
 (via (at 139.47023 82.516902) (size 0.6) (drill 0.3) (layers "F.Cu" "B.Cu") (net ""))
 (via (at 129.31023 72.356902) (size 0.6) (drill 0.3) (layers "F.Cu" "B.Cu") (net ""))
 (via (at 157.25023 107.916902) (size 0.6) (drill 0.3) (layers "F.Cu" "B.Cu") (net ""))
 (via (at 157.25023 105.376902) (size 0.6) (drill 0.3) (layers "F.Cu" "B.Cu") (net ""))
 (via (at 134.39023 74.896902) (size 0.6) (drill 0.3) (layers "F.Cu" "B.Cu") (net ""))
 (via (at 139.47023 97.756902) (size 0.6) (drill 0.3) (layers "F.Cu" "B.Cu") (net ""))
 (via (at 139.47023 125.696902) (size 0.6) (drill 0.3) (layers "F.Cu" "B.Cu") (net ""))
 (via (at 144.55023 107.916902) (size 0.6) (drill 0.3) (layers "F.Cu" "B.Cu") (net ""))
 (via (at 157.25023 110.456902) (size 0.6) (drill 0.3) (layers "F.Cu" "B.Cu") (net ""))
 (via (at 157.25023 118.076902) (size 0.6) (drill 0.3) (layers "F.Cu" "B.Cu") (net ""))
 (via (at 126.77023 82.516902) (size 0.6) (drill 0.3) (layers "F.Cu" "B.Cu") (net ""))
 (via (at 139.47023 74.896902) (size 0.6) (drill 0.3) (layers "F.Cu" "B.Cu") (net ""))
 (via (at 157.25023 72.356902) (size 0.6) (drill 0.3) (layers "F.Cu" "B.Cu") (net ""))
 (via (at 131.85023 67.276902) (size 0.6) (drill 0.3) (layers "F.Cu" "B.Cu") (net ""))
 (via (at 131.85023 69.816902) (size 0.6) (drill 0.3) (layers "F.Cu" "B.Cu") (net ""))
 (via (at 152.17023 125.696902) (size 0.6) (drill 0.3) (layers "F.Cu" "B.Cu") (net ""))
 (segment (start 142.01023 97.756902) (end 139.47023 97.756902) (width 0.2) (layer "B.Cu") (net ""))
 (segment (start 134.39023 79.976902) (end 136.505966 77.861166) (width 0.2) (layer "B.Cu") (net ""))
 (segment (start 154.71023 118.076902) (end 154.71023 120.616902) (width 0.2) (layer "B.Cu") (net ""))
 (segment (start 149.63023 90.136902) (end 142.01023 90.136902) (width 0.2) (layer "B.Cu") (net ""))
 (segment (start 126.77023 90.136902) (end 125.38023 90.136902) (width 0.2) (layer "B.Cu") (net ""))
 (segment (start 134.39023 100.296902) (end 140.86023 100.296902) (width 0.2) (layer "B.Cu") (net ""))
 (segment (start 144.55023 110.456902) (end 142.01023 110.456902) (width 0.2) (layer "B.Cu") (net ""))
 (segment (start 134.39023 87.596902) (end 134.39023 79.976902) (width 0.2) (layer "B.Cu") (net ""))
 (segment (start 159.79023 82.516902) (end 152.17023 82.516902) (width 0.2) (layer "B.Cu") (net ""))
 (segment (start 157.25023 110.456902) (end 159.79023 110.456902) (width 0.2) (layer "B.Cu") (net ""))
 (segment (start 157.25023 107.916902) (end 159.79023 107.916902) (width 0.2) (layer "B.Cu") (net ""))
 (segment (start 142.01023 85.056902) (end 140.62023 85.056902) (width 0.2) (layer "B.Cu") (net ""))
 (segment (start 157.25023 118.076902) (end 159.79023 118.076902) (width 0.2) (layer "B.Cu") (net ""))
 (segment (start 154.71023 102.836902) (end 154.71023 92.676902) (width 0.2) (layer "B.Cu") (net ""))
 (segment (start 157.25023 105.376902) (end 159.79023 105.376902) (width 0.2) (layer "B.Cu") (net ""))
 (segment (start 144.55023 92.676902) (end 142.01023 92.676902) (width 0.2) (layer "B.Cu") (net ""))
 (segment (start 124.23023 87.596902) (end 131.85023 87.596902) (width 0.2) (layer "B.Cu") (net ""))
 (segment (start 129.31023 72.356902) (end 134.39023 72.356902) (width 0.2) (layer "B.Cu") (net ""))
 (segment (start 144.55023 107.916902) (end 142.01023 107.916902) (width 0.2) (layer "B.Cu") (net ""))
 (segment (start 124.23023 74.896902) (end 134.39023 74.896902) (width 0.2) (layer "B.Cu") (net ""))
 (segment (start 124.23023 77.436902) (end 129.31023 77.436902) (width 0.2) (layer "B.Cu") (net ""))
 (segment (start 144.55023 120.616902) (end 142.01023 120.616902) (width 0.2) (layer "B.Cu") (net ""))
 (segment (start 142.01023 82.516902) (end 140.62023 82.516902) (width 0.2) (layer "B.Cu") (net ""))
 (segment (start 131.85023 67.276902) (end 131.85023 69.816902) (width 0.2) (layer "B.Cu") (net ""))
 (segment (start 136.93023 64.736902) (end 136.93023 77.436902) (width 0.2) (layer "B.Cu") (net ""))
 (segment (start 144.55023 105.376902) (end 142.01023 105.376902) (width 0.2) (layer "B.Cu") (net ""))
 (segment (start 139.47023 72.356902) (end 142.01023 72.356902) (width 0.2) (layer "B.Cu") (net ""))
 (segment (start 126.77023 82.516902) (end 124.23023 82.516902) (width 0.2) (layer "B.Cu") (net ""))
 (segment (start 159.79023 72.356902) (end 157.25023 72.356902) (width 0.2) (layer "B.Cu") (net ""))
 (segment (start 147.09023 102.836902) (end 147.09023 92.676902) (width 0.2) (layer "B.Cu") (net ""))
 (segment (start 139.47023 125.696902) (end 139.47023 118.076902) (width 0.2) (layer "B.Cu") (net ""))
 (segment (start 139.47023 77.436902) (end 142.01023 77.436902) (width 0.2) (layer "B.Cu") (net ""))
 (segment (start 147.09023 118.076902) (end 147.09023 120.616902) (width 0.2) (layer "B.Cu") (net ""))
 (segment (start 134.39023 123.156902) (end 134.39023 120.616902) (width 0.2) (layer "B.Cu") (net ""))
 (segment (start 147.09023 69.816902) (end 147.09023 64.736902) (width 0.2) (layer "B.Cu") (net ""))
 (segment (start 152.17023 125.696902) (end 142.01023 125.696902) (width 0.2) (layer "B.Cu") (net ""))
 (segment (start 139.47023 74.896902) (end 142.01023 74.896902) (width 0.2) (layer "B.Cu") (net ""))
 (segment (start 157.25023 120.616902) (end 159.79023 120.616902) (width 0.2) (layer "B.Cu") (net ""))
 (segment (start 126.77023 85.056902) (end 124.23023 85.056902) (width 0.2) (layer "B.Cu") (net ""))
 (segment (start 154.71023 85.056902) (end 152.17023 85.056902) (width 0.2) (layer "B.Cu") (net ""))
 (segment (start 152.17023 69.816902) (end 152.17023 67.276902) (width 0.2) (layer "B.Cu") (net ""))
 (segment (start 144.55023 118.076902) (end 142.01023 118.076902) (width 0.2) (layer "B.Cu") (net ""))
 (segment (start 154.71023 92.676902) (end 159.79023 92.676902) (width 0.2) (layer "B.Cu") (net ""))
 (segment (start 142.01023 87.596902) (end 140.62023 87.596902) (width 0.2) (layer "B.Cu") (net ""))
 (segment (start 124.23023 64.736902) (end 136.93023 64.736902) (width 0.2) (layer "B.Cu") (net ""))
 (segment (start 124.23023 67.276902) (end 124.23023 64.736902) (width 0.2) (layer "B.Cu") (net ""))
 (segment (start 149.63023 85.056902) (end 148.09023 85.056902) (width 0.2) (layer "B.Cu") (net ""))
 (segment (start 144.55023 112.996902) (end 142.01023 112.996902) (width 0.2) (layer "B.Cu") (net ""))
 (segment (start 157.25023 112.996902) (end 159.79023 112.996902) (width 0.2) (layer "B.Cu") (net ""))
 (segment (start 157.25023 74.896902) (end 159.79023 74.896902) (width 0.2) (layer "B.Cu") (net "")))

